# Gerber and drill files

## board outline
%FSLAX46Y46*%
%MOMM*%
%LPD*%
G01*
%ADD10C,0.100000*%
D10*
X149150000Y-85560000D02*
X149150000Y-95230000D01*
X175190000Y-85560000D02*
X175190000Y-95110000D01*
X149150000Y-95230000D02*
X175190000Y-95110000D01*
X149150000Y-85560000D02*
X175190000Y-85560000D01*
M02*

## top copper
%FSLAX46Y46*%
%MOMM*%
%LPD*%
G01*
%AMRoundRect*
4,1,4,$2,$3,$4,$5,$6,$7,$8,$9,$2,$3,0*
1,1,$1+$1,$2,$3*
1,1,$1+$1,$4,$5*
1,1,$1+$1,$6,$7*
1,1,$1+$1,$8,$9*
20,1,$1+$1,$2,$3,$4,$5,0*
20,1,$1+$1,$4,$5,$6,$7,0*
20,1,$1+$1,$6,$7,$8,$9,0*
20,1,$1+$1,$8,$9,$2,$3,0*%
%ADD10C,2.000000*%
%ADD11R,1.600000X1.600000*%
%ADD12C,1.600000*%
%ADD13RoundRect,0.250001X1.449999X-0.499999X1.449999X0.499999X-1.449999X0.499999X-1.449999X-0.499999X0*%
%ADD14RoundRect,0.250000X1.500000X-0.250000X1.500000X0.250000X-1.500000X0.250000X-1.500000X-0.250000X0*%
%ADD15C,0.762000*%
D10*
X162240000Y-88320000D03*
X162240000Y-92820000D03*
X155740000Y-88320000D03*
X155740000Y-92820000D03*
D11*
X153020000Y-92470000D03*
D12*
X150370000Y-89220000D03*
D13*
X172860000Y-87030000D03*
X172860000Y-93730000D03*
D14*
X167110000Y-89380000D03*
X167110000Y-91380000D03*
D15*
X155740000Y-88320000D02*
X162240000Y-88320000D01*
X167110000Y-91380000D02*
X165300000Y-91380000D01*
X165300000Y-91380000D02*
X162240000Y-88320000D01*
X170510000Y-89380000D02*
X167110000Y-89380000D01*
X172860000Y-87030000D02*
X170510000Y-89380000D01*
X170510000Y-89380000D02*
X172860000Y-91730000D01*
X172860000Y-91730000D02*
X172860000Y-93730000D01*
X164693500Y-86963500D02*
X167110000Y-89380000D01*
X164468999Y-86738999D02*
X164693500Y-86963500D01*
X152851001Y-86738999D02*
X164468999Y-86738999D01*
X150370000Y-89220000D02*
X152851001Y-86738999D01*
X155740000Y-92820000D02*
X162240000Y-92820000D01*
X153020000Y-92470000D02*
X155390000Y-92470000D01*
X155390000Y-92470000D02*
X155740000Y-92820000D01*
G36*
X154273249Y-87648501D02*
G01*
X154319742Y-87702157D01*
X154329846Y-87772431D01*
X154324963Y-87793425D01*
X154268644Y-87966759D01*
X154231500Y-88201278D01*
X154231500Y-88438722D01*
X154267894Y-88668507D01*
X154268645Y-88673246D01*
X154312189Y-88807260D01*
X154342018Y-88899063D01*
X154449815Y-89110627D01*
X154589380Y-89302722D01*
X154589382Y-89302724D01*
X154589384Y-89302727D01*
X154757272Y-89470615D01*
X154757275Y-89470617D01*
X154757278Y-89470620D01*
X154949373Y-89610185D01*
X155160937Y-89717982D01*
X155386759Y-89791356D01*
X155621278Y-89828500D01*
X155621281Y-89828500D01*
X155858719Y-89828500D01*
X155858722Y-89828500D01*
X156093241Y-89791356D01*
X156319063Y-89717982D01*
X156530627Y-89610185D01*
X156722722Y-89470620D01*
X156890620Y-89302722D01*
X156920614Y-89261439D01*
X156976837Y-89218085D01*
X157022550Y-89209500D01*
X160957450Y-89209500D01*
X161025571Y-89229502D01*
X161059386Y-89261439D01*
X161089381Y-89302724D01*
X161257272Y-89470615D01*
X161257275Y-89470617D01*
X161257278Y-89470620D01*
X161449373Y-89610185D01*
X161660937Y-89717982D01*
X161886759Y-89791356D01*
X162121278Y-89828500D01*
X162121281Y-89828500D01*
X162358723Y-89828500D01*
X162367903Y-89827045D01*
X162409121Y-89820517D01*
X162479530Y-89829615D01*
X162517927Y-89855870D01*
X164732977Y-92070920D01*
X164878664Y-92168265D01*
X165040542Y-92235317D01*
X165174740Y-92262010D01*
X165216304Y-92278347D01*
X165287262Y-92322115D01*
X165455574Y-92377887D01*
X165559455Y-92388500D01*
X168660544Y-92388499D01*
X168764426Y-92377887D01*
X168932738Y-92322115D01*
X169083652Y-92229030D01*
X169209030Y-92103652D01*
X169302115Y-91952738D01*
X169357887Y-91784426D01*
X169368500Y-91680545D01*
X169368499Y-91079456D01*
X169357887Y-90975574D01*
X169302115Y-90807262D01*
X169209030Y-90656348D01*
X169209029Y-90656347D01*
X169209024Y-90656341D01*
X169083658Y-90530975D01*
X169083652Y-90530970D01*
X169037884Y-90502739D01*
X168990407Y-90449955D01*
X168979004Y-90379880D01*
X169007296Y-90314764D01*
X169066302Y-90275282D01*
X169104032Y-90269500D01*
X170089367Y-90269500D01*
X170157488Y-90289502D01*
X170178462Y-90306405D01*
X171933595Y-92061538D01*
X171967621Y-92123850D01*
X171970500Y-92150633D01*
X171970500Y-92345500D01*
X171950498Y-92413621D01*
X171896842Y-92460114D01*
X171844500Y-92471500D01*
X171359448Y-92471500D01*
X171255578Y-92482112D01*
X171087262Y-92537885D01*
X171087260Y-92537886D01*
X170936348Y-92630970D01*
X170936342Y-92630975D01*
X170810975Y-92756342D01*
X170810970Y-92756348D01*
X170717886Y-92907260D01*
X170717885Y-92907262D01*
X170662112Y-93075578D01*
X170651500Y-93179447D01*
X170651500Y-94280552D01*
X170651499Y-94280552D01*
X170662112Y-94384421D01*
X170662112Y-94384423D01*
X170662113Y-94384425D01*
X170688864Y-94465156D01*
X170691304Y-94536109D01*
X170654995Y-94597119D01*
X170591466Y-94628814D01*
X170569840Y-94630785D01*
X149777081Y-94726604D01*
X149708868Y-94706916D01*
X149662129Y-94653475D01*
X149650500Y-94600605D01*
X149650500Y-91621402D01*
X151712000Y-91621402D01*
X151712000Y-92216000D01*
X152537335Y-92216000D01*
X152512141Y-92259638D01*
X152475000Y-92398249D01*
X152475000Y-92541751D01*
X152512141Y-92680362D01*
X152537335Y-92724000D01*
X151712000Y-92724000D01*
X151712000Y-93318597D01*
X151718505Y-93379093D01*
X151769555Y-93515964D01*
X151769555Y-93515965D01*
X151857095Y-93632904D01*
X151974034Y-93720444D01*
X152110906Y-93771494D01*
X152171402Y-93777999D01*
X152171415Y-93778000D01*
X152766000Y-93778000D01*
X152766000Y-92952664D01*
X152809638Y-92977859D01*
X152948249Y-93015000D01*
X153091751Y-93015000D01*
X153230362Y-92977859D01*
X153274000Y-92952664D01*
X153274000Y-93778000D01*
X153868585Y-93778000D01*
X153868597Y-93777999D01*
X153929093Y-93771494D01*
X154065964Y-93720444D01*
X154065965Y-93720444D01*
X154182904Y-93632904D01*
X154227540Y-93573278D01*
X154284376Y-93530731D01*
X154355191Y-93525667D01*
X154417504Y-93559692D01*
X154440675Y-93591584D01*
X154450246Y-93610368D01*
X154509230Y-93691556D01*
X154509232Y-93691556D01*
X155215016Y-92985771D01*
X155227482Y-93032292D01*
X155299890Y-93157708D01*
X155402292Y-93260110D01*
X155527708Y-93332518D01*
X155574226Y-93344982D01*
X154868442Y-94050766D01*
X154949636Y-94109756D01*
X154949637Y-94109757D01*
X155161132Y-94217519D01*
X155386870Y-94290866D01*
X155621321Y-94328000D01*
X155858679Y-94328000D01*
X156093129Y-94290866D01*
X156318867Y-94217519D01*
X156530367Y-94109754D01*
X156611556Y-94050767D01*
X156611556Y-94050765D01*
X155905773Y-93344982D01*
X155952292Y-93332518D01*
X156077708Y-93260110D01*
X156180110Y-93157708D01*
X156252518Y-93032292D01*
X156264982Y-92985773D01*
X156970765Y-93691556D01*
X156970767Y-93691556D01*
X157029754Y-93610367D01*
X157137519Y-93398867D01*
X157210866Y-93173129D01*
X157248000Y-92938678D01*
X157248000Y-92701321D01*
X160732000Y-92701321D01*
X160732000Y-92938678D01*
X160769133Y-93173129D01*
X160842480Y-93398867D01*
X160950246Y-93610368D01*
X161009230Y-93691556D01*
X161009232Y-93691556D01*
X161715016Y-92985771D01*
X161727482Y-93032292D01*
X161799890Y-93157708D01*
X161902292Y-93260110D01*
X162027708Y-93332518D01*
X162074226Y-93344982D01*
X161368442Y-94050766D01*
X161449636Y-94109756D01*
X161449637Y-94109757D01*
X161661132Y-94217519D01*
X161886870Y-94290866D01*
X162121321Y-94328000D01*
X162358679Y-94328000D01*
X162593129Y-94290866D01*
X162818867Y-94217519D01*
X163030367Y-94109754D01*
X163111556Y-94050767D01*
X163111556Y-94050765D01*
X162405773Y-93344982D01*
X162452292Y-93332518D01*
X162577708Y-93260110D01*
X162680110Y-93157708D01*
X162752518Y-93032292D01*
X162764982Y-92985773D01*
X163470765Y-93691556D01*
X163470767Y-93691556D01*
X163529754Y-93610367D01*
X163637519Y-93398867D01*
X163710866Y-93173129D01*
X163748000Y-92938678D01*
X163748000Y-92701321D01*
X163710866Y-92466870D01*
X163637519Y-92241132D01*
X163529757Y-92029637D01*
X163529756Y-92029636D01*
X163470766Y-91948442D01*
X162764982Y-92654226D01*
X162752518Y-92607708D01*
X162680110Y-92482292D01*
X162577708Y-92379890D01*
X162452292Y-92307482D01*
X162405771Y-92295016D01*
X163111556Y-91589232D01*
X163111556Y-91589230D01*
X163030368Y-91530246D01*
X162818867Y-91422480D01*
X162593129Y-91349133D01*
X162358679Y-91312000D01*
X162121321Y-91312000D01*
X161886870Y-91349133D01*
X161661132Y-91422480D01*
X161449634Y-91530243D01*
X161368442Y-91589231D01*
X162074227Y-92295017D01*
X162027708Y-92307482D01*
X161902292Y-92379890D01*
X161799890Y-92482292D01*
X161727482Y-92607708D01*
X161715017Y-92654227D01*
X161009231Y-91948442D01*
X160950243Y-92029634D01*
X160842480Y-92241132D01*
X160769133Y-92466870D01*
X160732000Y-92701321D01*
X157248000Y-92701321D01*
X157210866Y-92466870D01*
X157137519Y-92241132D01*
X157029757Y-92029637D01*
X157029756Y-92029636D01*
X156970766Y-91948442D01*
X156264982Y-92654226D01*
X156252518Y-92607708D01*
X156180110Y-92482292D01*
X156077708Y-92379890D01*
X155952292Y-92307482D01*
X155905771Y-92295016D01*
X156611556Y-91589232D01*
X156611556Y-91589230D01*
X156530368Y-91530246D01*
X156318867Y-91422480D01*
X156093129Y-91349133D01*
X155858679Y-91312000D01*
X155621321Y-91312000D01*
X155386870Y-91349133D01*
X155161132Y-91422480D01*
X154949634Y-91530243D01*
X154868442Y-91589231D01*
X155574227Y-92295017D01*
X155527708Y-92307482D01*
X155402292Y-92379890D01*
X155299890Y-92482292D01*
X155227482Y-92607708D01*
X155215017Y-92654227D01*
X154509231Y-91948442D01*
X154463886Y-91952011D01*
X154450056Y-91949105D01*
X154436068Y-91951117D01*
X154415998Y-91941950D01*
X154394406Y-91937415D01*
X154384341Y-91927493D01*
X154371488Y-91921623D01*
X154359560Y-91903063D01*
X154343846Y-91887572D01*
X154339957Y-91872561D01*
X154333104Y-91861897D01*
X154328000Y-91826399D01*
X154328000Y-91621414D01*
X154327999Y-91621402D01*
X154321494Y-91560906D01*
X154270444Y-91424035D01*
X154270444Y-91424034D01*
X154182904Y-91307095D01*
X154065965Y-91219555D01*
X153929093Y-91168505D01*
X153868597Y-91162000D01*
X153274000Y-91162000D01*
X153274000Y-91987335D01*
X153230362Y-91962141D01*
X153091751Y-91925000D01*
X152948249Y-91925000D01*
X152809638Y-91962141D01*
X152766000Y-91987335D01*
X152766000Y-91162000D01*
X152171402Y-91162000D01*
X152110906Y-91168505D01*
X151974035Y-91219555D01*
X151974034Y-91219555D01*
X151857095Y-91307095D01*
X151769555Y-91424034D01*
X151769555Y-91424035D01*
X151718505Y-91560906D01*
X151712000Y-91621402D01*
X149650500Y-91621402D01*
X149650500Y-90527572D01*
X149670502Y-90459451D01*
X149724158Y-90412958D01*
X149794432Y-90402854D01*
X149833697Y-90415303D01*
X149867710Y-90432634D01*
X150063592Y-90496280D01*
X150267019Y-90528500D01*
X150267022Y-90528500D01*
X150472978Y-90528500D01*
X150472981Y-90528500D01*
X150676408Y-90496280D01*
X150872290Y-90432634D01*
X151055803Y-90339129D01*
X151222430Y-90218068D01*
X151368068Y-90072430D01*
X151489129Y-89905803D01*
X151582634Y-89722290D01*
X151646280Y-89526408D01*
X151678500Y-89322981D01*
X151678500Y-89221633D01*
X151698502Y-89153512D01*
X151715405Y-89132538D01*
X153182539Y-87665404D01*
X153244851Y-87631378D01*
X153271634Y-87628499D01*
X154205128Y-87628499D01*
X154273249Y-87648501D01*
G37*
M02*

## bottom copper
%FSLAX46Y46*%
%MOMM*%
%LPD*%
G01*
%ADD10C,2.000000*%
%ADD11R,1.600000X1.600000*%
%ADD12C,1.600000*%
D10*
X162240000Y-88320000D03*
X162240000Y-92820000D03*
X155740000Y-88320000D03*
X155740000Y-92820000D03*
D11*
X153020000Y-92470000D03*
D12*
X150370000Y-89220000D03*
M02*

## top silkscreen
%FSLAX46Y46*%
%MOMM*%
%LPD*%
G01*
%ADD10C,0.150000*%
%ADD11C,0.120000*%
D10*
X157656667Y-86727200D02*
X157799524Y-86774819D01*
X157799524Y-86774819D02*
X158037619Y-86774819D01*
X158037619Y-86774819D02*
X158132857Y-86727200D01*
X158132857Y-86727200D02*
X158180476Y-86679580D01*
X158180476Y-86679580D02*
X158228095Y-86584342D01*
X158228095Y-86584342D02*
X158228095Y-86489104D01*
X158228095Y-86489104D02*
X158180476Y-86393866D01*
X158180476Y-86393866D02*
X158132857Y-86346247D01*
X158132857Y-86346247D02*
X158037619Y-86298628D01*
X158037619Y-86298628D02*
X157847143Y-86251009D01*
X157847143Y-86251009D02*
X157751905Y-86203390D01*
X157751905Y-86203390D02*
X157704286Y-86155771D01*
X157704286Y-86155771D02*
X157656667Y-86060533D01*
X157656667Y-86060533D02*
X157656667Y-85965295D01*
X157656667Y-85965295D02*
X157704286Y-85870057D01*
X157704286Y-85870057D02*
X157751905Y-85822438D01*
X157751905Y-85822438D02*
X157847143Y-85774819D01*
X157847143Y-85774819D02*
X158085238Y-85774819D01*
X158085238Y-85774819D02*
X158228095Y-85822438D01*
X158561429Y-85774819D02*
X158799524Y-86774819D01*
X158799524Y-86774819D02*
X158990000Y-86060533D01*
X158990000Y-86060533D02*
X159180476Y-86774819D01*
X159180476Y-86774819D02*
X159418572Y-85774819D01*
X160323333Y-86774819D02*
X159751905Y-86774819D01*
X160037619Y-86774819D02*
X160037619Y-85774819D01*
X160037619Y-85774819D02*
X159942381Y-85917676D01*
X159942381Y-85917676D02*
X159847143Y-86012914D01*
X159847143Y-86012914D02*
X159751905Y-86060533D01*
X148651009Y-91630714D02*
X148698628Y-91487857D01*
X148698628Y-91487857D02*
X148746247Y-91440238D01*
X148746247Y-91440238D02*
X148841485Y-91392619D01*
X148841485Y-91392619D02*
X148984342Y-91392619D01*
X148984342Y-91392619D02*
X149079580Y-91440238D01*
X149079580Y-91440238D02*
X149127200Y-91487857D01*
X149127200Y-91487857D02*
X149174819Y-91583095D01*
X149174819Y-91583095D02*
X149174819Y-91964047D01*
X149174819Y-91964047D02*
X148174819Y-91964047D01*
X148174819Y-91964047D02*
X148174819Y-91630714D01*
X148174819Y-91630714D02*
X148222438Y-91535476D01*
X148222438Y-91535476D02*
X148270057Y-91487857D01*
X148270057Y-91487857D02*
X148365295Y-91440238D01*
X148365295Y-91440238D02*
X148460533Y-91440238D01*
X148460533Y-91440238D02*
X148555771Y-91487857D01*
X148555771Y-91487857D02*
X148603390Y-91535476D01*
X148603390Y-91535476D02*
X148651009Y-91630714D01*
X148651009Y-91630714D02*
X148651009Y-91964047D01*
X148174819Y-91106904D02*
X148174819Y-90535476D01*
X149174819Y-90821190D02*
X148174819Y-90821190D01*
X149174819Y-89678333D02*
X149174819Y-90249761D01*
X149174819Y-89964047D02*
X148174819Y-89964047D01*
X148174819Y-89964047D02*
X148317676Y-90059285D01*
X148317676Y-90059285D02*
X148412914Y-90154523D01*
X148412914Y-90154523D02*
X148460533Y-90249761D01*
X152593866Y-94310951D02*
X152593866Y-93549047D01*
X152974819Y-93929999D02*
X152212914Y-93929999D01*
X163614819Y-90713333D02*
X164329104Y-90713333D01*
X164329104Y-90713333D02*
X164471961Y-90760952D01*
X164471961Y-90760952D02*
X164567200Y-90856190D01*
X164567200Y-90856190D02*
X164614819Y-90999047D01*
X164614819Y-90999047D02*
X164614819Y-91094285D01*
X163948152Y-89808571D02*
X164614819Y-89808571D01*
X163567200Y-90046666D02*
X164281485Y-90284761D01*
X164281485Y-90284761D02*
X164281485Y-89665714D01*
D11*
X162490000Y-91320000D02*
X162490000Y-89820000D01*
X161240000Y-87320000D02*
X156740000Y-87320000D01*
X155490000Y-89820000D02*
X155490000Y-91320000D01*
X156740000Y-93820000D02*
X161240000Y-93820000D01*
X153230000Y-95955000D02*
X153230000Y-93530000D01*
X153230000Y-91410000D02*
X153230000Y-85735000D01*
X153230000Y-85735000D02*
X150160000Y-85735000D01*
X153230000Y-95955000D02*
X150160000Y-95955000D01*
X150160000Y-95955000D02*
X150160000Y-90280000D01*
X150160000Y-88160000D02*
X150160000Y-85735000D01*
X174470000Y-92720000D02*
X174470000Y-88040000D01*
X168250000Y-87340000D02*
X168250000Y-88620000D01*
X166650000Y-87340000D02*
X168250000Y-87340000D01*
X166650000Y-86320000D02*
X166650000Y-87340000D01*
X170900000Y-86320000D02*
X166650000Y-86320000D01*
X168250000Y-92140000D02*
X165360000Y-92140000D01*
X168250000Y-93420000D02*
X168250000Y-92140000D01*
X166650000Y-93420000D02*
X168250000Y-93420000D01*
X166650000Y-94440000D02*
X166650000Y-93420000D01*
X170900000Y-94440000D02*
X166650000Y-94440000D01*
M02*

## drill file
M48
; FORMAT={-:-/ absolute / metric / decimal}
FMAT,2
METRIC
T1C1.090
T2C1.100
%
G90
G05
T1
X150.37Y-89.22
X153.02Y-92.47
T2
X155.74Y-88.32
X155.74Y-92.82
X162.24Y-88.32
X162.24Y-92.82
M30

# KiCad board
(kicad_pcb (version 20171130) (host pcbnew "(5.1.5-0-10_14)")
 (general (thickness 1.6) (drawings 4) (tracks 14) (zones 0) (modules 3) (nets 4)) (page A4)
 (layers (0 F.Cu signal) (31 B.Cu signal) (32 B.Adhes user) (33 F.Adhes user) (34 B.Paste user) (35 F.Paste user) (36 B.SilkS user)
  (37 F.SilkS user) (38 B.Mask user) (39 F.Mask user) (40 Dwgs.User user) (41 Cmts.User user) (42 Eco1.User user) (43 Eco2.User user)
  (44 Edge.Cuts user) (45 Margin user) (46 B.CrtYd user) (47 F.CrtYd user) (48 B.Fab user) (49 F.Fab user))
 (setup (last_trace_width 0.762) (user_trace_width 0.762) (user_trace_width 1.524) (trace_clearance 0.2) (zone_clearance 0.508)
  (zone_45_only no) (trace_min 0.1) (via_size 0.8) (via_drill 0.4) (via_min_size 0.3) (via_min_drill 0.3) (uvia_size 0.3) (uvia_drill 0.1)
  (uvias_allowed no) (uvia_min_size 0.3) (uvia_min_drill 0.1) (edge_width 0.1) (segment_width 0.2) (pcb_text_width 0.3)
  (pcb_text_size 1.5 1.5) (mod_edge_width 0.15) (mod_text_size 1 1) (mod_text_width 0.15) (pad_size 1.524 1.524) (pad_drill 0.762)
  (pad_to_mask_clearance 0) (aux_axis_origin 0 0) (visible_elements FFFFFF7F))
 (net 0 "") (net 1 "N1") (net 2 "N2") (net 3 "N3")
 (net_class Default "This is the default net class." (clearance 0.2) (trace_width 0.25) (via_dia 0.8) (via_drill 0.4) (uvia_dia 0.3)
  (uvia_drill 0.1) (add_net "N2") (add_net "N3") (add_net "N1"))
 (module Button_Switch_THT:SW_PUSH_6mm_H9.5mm (layer F.Cu) (at 155.74 88.32)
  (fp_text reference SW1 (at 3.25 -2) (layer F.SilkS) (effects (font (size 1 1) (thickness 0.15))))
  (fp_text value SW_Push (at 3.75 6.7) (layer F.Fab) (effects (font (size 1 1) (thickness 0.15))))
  (fp_line (start 6.75 3) (end 6.75 1.5) (layer F.SilkS) (width 0.12))
  (fp_line (start 5.5 -1) (end 1 -1) (layer F.SilkS) (width 0.12))
  (fp_line (start -0.25 1.5) (end -0.25 3) (layer F.SilkS) (width 0.12))
  (fp_line (start 1 5.5) (end 5.5 5.5) (layer F.SilkS) (width 0.12))
  (pad 1 thru_hole circle (at 6.5 0 90) (size 2 2) (drill 1.1) (layers *.Cu *.Mask) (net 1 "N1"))
  (pad 2 thru_hole circle (at 6.5 4.5 90) (size 2 2) (drill 1.1) (layers *.Cu *.Mask) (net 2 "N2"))
  (pad 1 thru_hole circle (at 0 0 90) (size 2 2) (drill 1.1) (layers *.Cu *.Mask) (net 1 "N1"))
  (pad 2 thru_hole circle (at 0 4.5 90) (size 2 2) (drill 1.1) (layers *.Cu *.Mask) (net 2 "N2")))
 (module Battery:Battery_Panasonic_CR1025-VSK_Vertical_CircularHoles (layer F.Cu) (at 153.02 92.47 90)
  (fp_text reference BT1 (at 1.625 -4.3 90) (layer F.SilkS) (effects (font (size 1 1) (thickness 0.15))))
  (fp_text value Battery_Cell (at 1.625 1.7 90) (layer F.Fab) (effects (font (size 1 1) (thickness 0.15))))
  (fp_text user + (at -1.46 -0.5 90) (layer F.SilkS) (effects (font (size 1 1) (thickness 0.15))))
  (fp_line (start -3.485 0.21) (end -1.06 0.21) (layer F.SilkS) (width 0.12))
  (fp_line (start 1.06 0.21) (end 6.735 0.21) (layer F.SilkS) (width 0.12))
  (fp_line (start 6.735 0.21) (end 6.735 -2.86) (layer F.SilkS) (width 0.12))
  (fp_line (start -3.485 0.21) (end -3.485 -2.86) (layer F.SilkS) (width 0.12))
  (fp_line (start -3.485 -2.86) (end 2.19 -2.86) (layer F.SilkS) (width 0.12))
  (fp_line (start 4.31 -2.86) (end 6.735 -2.86) (layer F.SilkS) (width 0.12))
  (pad 1 thru_hole rect (at 0 0 90) (size 1.6 1.6) (drill 1.09) (layers *.Cu *.Mask) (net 2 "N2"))
  (pad 2 thru_hole circle (at 3.25 -2.65 90) (size 1.6 1.6) (drill 1.09) (layers *.Cu *.Mask) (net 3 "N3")))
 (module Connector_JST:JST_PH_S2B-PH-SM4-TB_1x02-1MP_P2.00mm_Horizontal (layer F.Cu) (at 169.96 90.38 90)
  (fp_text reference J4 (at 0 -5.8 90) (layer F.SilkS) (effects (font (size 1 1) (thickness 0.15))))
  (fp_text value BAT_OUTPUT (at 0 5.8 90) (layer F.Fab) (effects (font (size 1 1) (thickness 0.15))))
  (fp_line (start -2.34 4.51) (end 2.34 4.51) (layer F.SilkS) (width 0.12))
  (fp_line (start 3.04 -1.71) (end 1.76 -1.71) (layer F.SilkS) (width 0.12))
  (fp_line (start 3.04 -3.31) (end 3.04 -1.71) (layer F.SilkS) (width 0.12))
  (fp_line (start 4.06 -3.31) (end 3.04 -3.31) (layer F.SilkS) (width 0.12))
  (fp_line (start 4.06 0.94) (end 4.06 -3.31) (layer F.SilkS) (width 0.12))
  (fp_line (start -1.76 -1.71) (end -1.76 -4.6) (layer F.SilkS) (width 0.12))
  (fp_line (start -3.04 -1.71) (end -1.76 -1.71) (layer F.SilkS) (width 0.12))
  (fp_line (start -3.04 -3.31) (end -3.04 -1.71) (layer F.SilkS) (width 0.12))
  (fp_line (start -4.06 -3.31) (end -3.04 -3.31) (layer F.SilkS) (width 0.12))
  (fp_line (start -4.06 0.94) (end -4.06 -3.31) (layer F.SilkS) (width 0.12))
  (pad MP smd roundrect (at 3.35 2.9 90) (size 1.5 3.4) (layers F.Cu F.Paste F.Mask) (roundrect_rratio 0.166667) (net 3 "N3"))
  (pad MP smd roundrect (at -3.35 2.9 90) (size 1.5 3.4) (layers F.Cu F.Paste F.Mask) (roundrect_rratio 0.166667) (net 3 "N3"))
  (pad 2 smd roundrect (at 1 -2.85 90) (size 1 3.5) (layers F.Cu F.Paste F.Mask) (roundrect_rratio 0.25) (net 3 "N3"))
  (pad 1 smd roundrect (at -1 -2.85 90) (size 1 3.5) (layers F.Cu F.Paste F.Mask) (roundrect_rratio 0.25) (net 1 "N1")))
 (gr_line (start 149.15 85.56) (end 149.15 95.23) (layer Edge.Cuts) (width 0.1))
 (gr_line (start 175.19 85.56) (end 175.19 95.11) (layer Edge.Cuts) (width 0.1))
 (gr_line (start 149.15 95.23) (end 175.19 95.11) (layer Edge.Cuts) (width 0.1))
 (gr_line (start 149.15 85.56) (end 175.19 85.56) (layer Edge.Cuts) (width 0.1))
 (segment (start 155.74 88.32) (end 162.24 88.32) (width 0.762) (layer F.Cu) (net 1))
 (segment (start 167.11 91.38) (end 165.3 91.38) (width 0.762) (layer F.Cu) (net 1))
 (segment (start 165.3 91.38) (end 162.24 88.32) (width 0.762) (layer F.Cu) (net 1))
 (segment (start 170.51 89.38) (end 167.11 89.38) (width 0.762) (layer F.Cu) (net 3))
 (segment (start 172.86 87.03) (end 170.51 89.38) (width 0.762) (layer F.Cu) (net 3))
 (segment (start 170.51 89.38) (end 172.86 91.73) (width 0.762) (layer F.Cu) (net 3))
 (segment (start 172.86 91.73) (end 172.86 93.73) (width 0.762) (layer F.Cu) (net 3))
 (segment (start 164.6935 86.9635) (end 167.11 89.38) (width 0.762) (layer F.Cu) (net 3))
 (segment (start 164.468999 86.738999) (end 164.6935 86.9635) (width 0.762) (layer F.Cu) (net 3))
 (segment (start 152.851001 86.738999) (end 164.468999 86.738999) (width 0.762) (layer F.Cu) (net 3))
 (segment (start 150.37 89.22) (end 152.851001 86.738999) (width 0.762) (layer F.Cu) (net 3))
 (segment (start 155.74 92.82) (end 162.24 92.82) (width 0.762) (layer F.Cu) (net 2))
 (segment (start 153.02 92.47) (end 155.39 92.47) (width 0.762) (layer F.Cu) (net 2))
 (segment (start 155.39 92.47) (end 155.74 92.82) (width 0.762) (layer F.Cu) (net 2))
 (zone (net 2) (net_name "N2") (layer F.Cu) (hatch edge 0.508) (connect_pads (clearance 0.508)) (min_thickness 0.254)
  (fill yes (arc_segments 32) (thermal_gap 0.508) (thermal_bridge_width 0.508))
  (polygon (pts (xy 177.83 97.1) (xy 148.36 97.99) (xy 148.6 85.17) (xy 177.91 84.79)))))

